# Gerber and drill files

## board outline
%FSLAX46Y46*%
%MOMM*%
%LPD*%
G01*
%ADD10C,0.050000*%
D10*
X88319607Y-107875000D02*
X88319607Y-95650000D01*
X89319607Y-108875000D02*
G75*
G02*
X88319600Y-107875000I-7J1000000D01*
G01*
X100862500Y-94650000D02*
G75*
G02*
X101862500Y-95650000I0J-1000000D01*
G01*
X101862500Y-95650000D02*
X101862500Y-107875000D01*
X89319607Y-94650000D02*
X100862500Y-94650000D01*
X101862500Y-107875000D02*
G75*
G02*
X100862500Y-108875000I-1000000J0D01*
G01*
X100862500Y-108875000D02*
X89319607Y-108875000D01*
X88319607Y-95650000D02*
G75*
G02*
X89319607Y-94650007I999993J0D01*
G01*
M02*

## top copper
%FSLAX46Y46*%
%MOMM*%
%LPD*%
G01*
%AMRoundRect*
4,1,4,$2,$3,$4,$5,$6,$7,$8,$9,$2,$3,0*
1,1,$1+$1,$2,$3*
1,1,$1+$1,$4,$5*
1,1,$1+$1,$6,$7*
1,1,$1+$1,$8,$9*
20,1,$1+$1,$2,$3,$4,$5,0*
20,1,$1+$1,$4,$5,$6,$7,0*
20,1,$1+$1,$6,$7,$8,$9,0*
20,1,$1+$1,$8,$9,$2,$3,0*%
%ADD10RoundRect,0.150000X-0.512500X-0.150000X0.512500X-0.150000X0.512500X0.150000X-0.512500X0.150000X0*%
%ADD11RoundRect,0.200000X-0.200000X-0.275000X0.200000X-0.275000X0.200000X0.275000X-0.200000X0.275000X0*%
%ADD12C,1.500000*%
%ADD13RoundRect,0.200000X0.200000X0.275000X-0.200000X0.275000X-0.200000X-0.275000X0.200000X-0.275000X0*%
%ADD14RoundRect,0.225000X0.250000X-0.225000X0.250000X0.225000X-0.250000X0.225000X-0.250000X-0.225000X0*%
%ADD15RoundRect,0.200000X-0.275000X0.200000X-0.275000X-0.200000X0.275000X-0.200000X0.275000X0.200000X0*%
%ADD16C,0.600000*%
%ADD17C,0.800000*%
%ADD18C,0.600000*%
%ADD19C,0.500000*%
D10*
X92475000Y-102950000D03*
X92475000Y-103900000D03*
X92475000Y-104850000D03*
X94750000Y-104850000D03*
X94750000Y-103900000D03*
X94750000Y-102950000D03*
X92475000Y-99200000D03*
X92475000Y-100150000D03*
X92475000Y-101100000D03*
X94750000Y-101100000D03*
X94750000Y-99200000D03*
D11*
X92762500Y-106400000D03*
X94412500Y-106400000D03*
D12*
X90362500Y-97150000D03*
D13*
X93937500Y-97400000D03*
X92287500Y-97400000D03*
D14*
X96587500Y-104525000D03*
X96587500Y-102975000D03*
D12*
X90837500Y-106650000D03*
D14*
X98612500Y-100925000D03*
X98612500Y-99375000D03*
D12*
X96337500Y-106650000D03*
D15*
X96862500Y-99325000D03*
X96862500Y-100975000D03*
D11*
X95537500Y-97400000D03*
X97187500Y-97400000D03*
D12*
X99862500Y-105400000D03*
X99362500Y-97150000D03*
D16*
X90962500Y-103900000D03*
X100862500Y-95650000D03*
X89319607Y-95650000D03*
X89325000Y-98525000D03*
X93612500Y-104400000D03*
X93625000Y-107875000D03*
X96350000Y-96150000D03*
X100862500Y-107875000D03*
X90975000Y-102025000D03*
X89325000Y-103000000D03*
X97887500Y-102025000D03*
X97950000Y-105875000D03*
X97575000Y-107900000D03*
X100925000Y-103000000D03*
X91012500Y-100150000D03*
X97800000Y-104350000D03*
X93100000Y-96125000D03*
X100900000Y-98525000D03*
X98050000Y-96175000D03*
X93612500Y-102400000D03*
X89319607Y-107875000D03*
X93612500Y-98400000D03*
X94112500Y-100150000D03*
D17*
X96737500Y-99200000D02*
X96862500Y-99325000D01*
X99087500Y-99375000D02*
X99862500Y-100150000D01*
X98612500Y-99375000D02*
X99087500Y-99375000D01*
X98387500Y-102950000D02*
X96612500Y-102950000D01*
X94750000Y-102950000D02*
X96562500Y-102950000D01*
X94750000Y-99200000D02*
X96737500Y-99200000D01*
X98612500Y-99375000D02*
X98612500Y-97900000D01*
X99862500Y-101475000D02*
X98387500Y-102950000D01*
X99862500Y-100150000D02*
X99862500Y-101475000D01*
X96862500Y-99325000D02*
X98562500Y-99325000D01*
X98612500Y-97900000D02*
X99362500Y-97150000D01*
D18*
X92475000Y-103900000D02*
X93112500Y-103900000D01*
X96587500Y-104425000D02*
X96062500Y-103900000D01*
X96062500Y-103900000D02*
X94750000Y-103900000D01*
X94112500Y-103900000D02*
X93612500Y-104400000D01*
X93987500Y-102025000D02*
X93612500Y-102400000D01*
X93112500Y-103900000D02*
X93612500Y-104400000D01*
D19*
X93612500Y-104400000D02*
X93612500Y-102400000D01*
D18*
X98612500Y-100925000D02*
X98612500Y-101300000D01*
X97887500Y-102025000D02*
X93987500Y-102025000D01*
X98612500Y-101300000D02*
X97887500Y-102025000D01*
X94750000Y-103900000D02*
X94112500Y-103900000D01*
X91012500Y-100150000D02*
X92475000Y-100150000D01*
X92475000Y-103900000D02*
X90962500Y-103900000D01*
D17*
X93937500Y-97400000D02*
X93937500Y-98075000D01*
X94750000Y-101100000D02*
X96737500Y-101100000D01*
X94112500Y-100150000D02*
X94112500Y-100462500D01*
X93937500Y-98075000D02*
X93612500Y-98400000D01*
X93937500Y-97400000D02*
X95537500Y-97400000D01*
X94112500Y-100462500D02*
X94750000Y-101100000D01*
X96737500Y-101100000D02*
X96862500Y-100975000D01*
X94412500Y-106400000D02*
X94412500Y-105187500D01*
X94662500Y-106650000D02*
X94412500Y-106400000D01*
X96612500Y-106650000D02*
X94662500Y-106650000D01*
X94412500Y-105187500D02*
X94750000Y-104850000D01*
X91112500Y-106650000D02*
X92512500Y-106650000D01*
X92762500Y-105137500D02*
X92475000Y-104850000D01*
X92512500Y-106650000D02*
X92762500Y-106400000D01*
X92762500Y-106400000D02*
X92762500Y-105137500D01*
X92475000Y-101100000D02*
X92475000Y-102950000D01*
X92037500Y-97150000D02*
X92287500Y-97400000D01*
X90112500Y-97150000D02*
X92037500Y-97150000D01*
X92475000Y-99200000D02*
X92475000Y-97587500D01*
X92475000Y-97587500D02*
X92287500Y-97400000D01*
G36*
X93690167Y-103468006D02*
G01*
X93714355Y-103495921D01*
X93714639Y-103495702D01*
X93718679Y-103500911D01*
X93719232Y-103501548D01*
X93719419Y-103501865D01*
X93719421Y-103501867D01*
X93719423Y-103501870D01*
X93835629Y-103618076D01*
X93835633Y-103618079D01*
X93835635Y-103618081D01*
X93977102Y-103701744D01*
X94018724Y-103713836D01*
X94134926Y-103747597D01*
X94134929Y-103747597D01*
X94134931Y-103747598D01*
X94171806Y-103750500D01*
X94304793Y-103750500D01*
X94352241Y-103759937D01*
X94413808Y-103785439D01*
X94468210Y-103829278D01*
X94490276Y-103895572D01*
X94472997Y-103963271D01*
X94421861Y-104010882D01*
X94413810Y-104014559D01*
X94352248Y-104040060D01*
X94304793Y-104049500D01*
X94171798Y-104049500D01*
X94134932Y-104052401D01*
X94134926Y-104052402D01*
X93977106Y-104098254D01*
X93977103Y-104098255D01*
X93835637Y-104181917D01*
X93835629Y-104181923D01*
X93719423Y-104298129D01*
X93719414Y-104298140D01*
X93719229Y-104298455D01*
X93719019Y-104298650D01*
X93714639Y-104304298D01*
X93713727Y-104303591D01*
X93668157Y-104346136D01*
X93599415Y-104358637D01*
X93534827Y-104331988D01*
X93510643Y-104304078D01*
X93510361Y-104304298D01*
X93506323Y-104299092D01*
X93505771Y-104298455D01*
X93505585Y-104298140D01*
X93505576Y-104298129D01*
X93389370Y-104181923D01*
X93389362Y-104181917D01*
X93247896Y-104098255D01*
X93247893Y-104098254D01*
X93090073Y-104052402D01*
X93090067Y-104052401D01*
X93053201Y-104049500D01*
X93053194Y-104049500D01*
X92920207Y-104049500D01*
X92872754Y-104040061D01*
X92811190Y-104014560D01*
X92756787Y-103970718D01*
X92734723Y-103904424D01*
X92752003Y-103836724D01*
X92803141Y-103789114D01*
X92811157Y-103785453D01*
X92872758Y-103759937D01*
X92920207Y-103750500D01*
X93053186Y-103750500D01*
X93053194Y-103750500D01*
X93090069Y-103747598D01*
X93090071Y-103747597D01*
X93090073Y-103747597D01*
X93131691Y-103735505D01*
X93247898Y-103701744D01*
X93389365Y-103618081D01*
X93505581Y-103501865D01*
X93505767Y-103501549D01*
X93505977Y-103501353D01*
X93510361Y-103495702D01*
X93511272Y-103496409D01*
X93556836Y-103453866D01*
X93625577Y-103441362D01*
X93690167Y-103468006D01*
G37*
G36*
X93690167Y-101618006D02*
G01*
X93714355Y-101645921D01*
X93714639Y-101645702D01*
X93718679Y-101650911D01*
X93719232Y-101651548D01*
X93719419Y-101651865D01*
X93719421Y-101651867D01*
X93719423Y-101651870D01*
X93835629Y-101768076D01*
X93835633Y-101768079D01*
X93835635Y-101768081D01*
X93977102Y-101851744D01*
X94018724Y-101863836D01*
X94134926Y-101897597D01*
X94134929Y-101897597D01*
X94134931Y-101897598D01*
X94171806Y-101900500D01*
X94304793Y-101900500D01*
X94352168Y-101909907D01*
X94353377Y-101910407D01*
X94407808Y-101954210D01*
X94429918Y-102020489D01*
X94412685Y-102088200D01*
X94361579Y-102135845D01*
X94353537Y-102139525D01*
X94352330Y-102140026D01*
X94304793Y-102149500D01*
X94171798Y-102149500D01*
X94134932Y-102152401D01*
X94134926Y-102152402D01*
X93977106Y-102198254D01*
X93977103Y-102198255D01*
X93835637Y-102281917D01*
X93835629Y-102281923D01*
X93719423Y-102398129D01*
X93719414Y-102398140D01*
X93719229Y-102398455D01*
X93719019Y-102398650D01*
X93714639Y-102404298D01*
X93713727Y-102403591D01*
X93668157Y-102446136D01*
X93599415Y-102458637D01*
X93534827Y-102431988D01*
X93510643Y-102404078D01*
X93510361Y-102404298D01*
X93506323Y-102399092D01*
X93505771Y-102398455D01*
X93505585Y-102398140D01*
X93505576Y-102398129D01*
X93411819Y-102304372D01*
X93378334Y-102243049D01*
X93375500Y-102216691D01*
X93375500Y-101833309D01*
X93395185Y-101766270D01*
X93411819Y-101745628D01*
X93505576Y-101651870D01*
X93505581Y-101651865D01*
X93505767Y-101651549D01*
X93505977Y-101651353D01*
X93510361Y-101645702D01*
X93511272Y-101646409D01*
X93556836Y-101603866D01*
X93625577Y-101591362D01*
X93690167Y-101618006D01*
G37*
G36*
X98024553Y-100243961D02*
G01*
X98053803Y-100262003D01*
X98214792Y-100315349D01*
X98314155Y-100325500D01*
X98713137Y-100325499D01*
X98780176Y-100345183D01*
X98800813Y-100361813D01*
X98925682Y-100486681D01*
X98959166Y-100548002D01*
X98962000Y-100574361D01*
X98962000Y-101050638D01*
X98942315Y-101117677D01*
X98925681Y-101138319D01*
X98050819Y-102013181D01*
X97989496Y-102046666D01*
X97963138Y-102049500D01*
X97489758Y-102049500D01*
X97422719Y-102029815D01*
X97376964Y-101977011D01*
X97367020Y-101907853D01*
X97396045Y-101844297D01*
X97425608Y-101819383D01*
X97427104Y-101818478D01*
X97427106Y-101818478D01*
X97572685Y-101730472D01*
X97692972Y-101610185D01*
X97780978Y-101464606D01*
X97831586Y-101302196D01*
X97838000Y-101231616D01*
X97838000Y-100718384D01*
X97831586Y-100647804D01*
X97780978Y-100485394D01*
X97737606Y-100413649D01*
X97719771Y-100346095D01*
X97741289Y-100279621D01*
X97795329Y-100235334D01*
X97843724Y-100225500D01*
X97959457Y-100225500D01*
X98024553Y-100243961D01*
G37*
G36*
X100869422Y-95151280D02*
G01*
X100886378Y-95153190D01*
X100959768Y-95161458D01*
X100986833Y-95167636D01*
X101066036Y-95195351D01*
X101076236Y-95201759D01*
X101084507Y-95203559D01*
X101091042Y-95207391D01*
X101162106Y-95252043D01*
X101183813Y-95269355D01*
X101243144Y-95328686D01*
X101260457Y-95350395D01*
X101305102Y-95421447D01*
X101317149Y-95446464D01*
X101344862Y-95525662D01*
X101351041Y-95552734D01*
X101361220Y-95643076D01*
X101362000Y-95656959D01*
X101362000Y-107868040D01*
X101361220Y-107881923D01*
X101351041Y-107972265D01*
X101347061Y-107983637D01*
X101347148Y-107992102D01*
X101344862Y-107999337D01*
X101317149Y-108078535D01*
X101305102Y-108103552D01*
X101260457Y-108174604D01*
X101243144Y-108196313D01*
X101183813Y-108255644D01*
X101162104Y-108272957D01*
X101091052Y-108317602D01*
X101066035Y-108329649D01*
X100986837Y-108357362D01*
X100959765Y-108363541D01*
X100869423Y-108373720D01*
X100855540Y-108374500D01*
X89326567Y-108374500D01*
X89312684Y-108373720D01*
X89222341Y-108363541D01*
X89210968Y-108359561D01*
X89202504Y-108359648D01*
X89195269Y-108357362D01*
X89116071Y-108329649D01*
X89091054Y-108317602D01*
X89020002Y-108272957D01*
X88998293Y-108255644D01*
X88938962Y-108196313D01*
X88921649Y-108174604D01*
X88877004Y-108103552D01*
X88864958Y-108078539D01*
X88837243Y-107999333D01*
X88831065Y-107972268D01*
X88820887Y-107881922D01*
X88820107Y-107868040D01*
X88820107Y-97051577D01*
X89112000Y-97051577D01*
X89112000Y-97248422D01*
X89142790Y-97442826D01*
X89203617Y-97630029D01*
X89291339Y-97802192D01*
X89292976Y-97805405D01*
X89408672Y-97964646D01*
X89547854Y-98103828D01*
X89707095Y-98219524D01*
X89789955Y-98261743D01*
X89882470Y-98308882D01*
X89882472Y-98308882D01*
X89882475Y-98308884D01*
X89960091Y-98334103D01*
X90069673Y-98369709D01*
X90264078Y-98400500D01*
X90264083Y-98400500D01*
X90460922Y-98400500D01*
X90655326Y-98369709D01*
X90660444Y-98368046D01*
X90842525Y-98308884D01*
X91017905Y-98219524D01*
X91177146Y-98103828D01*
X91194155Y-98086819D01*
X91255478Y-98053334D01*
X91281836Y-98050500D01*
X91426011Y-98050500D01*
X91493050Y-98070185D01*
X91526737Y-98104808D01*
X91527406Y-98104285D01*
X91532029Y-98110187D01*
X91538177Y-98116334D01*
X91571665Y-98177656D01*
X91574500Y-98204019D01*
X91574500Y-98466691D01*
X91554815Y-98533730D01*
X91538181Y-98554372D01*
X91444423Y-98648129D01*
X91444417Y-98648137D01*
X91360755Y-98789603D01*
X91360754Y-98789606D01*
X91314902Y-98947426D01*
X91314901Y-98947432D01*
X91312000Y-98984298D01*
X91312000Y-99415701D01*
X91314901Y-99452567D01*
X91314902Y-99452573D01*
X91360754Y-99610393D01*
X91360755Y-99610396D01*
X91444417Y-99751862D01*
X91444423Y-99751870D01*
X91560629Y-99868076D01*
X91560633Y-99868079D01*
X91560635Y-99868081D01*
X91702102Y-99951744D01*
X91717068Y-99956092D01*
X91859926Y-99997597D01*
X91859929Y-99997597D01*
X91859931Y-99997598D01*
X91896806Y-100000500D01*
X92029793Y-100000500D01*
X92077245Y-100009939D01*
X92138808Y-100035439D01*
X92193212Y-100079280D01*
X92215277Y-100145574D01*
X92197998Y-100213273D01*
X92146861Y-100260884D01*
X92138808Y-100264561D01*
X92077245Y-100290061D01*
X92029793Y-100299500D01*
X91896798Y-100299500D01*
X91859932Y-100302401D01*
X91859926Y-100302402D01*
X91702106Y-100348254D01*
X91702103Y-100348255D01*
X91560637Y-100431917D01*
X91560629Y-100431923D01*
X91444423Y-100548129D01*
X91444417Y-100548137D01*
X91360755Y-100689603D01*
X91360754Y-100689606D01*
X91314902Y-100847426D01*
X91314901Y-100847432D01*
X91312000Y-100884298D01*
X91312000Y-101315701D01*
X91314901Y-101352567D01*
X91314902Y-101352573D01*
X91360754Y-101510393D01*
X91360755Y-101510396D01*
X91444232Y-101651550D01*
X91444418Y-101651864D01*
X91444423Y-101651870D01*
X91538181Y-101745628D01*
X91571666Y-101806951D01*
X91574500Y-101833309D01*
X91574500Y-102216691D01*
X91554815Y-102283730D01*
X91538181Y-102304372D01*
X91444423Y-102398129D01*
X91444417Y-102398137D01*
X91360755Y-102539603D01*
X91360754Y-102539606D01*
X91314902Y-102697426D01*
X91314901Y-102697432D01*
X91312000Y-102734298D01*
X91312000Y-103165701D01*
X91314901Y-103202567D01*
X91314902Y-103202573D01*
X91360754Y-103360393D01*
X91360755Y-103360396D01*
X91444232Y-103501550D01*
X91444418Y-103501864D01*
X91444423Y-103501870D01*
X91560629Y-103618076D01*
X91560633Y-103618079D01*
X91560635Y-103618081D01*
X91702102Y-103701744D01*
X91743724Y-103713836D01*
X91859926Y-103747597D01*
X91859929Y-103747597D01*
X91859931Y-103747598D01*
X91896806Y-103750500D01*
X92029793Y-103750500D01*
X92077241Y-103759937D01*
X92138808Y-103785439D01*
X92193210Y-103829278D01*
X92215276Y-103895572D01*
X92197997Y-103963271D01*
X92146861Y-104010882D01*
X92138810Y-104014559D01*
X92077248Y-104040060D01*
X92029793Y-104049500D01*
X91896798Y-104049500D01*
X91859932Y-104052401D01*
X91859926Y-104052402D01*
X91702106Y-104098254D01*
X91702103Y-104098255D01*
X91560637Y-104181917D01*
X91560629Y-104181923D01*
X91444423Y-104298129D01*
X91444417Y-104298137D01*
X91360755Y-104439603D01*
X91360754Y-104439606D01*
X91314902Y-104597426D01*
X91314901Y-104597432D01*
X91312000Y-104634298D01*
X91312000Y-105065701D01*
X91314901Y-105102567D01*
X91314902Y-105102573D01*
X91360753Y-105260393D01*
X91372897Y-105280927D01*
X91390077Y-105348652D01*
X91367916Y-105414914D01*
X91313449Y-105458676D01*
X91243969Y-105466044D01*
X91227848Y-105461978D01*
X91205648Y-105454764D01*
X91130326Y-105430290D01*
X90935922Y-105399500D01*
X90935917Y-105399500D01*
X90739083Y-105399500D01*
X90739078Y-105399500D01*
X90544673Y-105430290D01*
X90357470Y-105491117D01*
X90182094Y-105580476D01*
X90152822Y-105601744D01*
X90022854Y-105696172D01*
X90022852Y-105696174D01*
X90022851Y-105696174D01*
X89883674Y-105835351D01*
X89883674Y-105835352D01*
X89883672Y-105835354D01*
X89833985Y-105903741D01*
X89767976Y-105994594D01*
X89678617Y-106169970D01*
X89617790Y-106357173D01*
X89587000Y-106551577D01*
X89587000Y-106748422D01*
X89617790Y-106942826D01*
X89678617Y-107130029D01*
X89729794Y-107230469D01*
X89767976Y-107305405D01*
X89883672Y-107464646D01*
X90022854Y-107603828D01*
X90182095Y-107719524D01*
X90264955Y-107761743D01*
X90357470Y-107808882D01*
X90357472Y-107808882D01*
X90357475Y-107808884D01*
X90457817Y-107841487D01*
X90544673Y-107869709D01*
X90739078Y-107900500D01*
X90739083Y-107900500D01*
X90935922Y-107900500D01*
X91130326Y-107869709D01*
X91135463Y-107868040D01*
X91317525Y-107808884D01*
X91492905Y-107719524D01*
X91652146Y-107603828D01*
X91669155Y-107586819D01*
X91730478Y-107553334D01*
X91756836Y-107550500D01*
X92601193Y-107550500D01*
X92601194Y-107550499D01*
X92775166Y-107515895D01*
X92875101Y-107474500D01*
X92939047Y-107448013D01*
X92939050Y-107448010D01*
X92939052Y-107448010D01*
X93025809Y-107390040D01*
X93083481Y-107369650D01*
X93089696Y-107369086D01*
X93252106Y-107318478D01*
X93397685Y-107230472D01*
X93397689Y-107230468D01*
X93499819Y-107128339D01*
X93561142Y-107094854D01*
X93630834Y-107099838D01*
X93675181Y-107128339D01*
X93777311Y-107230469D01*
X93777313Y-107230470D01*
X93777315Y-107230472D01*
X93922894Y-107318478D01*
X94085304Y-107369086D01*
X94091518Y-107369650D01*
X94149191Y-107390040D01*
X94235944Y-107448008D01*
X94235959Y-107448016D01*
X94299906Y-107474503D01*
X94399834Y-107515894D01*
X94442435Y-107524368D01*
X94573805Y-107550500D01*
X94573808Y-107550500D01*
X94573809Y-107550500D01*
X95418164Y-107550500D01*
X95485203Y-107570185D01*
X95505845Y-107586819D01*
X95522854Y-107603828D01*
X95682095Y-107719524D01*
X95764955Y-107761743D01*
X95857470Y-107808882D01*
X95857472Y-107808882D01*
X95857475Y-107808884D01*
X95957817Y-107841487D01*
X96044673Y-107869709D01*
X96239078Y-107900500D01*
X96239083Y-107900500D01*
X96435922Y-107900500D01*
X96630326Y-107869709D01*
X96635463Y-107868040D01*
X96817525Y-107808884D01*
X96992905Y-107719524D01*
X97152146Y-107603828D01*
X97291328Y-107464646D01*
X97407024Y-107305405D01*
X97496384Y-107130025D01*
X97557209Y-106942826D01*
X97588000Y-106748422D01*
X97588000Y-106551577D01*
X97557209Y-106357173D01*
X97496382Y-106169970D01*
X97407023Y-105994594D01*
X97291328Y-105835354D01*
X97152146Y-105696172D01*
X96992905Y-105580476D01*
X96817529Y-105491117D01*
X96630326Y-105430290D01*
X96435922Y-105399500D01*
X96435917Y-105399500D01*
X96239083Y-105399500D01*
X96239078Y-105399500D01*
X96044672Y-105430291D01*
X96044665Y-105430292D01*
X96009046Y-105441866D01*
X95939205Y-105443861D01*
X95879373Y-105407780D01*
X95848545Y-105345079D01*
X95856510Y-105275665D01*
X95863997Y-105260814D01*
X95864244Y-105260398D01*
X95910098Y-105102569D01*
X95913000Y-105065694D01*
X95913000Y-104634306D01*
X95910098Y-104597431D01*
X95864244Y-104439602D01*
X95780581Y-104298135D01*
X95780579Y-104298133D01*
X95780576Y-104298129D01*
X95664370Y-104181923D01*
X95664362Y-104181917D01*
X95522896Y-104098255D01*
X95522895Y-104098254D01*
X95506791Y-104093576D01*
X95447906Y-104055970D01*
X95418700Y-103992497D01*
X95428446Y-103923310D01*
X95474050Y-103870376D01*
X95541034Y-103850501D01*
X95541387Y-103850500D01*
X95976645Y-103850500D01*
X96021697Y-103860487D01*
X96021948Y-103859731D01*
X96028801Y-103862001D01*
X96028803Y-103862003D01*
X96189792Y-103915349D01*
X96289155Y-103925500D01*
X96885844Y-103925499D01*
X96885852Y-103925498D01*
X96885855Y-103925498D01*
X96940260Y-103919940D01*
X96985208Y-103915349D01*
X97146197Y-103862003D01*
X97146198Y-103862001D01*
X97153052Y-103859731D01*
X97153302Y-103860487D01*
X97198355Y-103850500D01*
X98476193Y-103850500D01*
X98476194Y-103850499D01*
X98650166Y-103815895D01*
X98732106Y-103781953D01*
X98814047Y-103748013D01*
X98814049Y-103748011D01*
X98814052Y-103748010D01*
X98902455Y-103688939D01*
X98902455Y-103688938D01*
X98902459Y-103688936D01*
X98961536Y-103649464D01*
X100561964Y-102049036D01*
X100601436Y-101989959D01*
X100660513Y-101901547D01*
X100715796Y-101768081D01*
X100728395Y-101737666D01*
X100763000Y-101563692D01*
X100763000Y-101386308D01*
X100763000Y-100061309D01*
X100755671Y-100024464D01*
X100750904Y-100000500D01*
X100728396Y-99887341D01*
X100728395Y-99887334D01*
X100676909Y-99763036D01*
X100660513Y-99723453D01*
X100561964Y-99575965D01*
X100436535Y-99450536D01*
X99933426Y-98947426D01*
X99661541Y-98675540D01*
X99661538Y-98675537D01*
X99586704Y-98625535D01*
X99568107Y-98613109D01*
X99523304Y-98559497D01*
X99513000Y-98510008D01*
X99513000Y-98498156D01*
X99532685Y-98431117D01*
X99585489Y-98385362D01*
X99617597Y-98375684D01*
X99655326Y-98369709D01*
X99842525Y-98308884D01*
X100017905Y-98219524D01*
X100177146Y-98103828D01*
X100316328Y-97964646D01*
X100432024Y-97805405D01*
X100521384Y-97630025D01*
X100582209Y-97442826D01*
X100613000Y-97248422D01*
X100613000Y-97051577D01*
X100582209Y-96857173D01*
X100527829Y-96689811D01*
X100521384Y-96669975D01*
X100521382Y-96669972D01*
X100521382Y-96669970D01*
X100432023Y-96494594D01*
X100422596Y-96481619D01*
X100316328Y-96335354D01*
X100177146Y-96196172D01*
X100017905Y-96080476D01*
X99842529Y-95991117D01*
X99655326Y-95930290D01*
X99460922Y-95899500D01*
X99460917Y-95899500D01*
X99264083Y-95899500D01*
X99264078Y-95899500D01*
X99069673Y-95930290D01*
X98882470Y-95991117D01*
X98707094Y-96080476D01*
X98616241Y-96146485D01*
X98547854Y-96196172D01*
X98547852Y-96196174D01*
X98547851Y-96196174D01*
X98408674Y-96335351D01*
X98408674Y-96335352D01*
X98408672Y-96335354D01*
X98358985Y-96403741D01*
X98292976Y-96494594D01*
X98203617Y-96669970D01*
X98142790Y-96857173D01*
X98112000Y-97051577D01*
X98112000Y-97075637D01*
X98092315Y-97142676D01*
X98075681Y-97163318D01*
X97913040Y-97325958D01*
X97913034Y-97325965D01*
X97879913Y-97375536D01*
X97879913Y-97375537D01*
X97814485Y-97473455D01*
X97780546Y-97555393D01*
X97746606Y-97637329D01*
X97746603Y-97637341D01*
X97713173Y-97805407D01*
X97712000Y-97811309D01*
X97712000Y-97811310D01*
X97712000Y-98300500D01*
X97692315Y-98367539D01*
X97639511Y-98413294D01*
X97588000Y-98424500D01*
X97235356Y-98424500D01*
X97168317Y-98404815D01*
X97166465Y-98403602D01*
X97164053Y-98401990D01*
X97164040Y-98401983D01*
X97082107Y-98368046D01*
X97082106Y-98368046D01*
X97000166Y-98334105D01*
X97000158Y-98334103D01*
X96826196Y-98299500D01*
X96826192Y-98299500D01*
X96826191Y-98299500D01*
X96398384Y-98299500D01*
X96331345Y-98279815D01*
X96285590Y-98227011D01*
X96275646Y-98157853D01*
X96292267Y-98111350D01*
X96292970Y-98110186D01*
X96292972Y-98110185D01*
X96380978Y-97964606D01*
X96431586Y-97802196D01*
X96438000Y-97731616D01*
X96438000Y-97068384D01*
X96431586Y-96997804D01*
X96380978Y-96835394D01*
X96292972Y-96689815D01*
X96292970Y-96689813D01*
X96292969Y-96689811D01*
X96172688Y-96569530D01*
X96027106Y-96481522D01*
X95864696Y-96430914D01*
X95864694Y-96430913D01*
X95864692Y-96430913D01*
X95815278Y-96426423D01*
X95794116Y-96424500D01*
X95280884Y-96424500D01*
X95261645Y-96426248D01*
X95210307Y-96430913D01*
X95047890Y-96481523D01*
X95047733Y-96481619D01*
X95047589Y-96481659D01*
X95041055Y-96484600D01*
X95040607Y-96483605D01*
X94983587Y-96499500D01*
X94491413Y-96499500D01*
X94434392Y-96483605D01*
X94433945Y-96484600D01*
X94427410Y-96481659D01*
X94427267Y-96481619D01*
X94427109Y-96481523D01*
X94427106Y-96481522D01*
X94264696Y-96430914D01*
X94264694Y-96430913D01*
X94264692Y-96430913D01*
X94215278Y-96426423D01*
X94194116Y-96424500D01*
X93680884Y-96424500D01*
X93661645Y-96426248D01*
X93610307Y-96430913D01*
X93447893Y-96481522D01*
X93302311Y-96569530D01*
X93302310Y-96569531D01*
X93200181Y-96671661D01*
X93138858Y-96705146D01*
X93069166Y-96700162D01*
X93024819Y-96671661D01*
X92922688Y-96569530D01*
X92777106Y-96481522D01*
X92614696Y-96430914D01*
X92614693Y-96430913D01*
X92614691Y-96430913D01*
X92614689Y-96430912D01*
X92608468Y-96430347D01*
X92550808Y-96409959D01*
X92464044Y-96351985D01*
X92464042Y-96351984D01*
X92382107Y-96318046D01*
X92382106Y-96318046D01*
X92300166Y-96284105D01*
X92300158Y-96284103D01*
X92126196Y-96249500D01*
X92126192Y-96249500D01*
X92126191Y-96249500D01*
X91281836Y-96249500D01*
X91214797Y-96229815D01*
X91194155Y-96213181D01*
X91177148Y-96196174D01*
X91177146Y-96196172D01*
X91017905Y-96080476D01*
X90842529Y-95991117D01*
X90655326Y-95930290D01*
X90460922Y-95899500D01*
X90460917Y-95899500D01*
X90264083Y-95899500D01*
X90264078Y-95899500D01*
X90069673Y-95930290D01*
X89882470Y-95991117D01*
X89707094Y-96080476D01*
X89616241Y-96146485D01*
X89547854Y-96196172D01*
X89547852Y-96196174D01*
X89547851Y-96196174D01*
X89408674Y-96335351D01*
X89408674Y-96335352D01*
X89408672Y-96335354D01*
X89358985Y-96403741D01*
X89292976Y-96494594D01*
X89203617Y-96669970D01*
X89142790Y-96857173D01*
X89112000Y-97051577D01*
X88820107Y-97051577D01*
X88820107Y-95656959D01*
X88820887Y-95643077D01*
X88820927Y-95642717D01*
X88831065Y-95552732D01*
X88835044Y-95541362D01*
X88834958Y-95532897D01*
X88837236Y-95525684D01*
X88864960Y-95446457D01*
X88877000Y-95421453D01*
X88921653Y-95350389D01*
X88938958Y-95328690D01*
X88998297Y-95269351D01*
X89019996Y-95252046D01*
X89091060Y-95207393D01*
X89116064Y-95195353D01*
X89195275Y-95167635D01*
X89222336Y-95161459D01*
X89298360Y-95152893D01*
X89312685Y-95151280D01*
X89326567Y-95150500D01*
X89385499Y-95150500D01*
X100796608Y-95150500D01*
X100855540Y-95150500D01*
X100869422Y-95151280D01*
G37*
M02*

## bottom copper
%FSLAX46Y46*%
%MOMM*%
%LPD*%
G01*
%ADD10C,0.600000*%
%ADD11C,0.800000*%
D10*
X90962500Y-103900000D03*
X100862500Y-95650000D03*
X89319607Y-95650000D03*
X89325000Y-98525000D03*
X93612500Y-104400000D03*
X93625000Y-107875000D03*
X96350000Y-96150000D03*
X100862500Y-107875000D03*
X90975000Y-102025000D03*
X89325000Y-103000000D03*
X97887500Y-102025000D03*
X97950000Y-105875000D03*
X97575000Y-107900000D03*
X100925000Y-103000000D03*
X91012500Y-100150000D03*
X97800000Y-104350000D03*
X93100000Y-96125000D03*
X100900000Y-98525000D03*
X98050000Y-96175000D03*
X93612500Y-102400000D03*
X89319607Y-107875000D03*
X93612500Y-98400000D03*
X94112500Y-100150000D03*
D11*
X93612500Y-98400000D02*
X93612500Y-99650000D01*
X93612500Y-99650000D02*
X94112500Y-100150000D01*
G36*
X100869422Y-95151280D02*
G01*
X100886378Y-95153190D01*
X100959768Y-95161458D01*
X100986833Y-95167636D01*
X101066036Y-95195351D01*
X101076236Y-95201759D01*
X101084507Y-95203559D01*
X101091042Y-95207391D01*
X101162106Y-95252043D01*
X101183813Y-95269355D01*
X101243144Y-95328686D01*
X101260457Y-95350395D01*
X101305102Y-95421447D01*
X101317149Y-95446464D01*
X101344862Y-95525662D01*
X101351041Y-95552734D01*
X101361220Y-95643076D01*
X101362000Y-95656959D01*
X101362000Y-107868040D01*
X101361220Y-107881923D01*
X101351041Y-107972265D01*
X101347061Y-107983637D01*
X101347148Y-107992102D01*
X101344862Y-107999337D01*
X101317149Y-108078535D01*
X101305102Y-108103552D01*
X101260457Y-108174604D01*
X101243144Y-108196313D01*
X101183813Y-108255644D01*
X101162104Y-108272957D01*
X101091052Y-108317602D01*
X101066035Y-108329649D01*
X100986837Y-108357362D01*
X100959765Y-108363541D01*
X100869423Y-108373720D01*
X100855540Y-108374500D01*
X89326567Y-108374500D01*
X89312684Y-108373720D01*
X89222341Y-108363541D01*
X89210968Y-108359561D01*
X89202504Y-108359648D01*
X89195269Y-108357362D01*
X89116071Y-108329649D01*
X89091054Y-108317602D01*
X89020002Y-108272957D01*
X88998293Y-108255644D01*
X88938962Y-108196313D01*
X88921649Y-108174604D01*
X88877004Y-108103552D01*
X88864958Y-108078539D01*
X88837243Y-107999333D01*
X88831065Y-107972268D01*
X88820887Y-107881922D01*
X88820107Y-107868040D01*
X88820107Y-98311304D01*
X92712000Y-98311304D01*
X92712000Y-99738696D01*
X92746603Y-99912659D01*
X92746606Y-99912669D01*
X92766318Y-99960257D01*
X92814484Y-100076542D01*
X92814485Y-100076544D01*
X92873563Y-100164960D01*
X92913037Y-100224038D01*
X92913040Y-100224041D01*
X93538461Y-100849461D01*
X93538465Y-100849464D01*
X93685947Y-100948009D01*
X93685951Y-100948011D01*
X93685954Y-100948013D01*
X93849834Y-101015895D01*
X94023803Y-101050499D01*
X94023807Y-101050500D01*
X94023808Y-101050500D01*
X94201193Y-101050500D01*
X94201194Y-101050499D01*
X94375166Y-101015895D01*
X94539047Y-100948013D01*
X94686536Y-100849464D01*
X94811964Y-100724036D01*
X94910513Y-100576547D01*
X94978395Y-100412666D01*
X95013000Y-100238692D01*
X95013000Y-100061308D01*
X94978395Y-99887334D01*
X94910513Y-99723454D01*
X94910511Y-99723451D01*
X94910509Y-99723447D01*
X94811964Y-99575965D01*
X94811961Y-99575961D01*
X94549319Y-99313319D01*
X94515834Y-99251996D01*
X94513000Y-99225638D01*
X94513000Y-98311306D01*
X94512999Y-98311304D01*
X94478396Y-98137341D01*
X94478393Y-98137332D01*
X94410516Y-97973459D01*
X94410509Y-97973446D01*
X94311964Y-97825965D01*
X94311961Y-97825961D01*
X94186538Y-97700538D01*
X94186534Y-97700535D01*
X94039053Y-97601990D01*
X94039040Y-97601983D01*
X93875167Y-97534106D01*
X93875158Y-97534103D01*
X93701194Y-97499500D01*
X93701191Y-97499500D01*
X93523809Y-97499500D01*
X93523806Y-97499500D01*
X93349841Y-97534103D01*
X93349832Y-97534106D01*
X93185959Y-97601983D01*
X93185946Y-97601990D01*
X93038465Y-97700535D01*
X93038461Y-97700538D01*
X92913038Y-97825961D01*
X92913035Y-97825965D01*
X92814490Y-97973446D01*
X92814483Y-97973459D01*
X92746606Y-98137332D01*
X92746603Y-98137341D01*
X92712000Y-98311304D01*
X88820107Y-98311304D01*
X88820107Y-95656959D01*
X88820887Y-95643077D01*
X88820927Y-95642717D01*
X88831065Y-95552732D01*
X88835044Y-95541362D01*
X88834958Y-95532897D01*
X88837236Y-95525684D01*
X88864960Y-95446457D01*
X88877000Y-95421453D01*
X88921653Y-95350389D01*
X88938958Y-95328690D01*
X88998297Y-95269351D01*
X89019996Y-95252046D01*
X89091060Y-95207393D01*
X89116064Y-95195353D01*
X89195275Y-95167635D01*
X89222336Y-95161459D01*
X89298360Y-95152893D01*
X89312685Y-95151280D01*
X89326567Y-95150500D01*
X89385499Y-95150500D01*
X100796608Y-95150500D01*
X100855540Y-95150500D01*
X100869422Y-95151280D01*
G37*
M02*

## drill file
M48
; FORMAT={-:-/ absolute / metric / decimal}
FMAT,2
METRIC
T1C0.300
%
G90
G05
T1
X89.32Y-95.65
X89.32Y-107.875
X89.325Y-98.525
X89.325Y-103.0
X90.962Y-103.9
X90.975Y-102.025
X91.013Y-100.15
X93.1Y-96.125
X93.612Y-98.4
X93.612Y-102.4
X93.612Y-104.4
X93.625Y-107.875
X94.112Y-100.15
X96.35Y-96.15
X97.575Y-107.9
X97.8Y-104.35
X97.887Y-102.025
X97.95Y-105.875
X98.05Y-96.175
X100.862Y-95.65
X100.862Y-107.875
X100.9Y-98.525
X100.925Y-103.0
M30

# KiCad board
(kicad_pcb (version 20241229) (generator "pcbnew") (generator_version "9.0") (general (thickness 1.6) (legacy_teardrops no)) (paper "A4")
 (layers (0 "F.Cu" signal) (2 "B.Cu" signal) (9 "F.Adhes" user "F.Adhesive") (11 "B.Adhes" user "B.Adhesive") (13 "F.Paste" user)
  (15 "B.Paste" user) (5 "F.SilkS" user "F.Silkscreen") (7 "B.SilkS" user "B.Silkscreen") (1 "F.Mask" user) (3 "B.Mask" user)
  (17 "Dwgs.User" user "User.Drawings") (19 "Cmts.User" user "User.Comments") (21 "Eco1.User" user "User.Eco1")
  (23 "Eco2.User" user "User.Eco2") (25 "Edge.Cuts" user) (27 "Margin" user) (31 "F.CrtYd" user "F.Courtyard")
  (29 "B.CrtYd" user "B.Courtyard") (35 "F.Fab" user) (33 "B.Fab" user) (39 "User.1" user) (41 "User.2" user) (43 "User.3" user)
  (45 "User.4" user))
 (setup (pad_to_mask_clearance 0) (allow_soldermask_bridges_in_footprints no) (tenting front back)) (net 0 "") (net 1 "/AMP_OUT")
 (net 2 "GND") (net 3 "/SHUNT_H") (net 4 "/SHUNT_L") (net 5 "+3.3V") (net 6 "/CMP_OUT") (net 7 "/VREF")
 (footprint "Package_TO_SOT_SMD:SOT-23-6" (layer "F.Cu") (at 93.6125 103.9)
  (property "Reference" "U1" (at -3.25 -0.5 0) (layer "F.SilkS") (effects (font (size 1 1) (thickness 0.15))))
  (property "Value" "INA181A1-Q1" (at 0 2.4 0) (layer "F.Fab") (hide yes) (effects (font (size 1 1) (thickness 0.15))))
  (pad "1" smd roundrect (at -1.1375 -0.95) (size 1.325 0.6) (layers "F.Cu" "F.Mask" "F.Paste") (roundrect_rratio 0.25) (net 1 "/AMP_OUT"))
  (pad "2" smd roundrect (at -1.1375 0) (size 1.325 0.6) (layers "F.Cu" "F.Mask" "F.Paste") (roundrect_rratio 0.25) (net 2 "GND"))
  (pad "3" smd roundrect (at -1.1375 0.95) (size 1.325 0.6) (layers "F.Cu" "F.Mask" "F.Paste") (roundrect_rratio 0.25) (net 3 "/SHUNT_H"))
  (pad "4" smd roundrect (at 1.1375 0.95) (size 1.325 0.6) (layers "F.Cu" "F.Mask" "F.Paste") (roundrect_rratio 0.25) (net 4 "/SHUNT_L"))
  (pad "5" smd roundrect (at 1.1375 0) (size 1.325 0.6) (layers "F.Cu" "F.Mask" "F.Paste") (roundrect_rratio 0.25) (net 2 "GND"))
  (pad "6" smd roundrect (at 1.1375 -0.95) (size 1.325 0.6) (layers "F.Cu" "F.Mask" "F.Paste") (roundrect_rratio 0.25) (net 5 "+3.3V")))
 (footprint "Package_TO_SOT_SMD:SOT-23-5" (layer "F.Cu") (at 93.6125 100.15)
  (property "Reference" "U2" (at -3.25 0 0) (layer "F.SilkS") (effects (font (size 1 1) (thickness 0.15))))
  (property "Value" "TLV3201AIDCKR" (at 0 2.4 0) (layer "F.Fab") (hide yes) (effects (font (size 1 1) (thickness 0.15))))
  (pad "1" smd roundrect (at -1.1375 -0.95) (size 1.325 0.6) (layers "F.Cu" "F.Mask" "F.Paste") (roundrect_rratio 0.25) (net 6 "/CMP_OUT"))
  (pad "2" smd roundrect (at -1.1375 0) (size 1.325 0.6) (layers "F.Cu" "F.Mask" "F.Paste") (roundrect_rratio 0.25) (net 2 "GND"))
  (pad "3" smd roundrect (at -1.1375 0.95) (size 1.325 0.6) (layers "F.Cu" "F.Mask" "F.Paste") (roundrect_rratio 0.25) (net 1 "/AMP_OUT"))
  (pad "4" smd roundrect (at 1.1375 0.95) (size 1.325 0.6) (layers "F.Cu" "F.Mask" "F.Paste") (roundrect_rratio 0.25) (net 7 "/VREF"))
  (pad "5" smd roundrect (at 1.1375 -0.95) (size 1.325 0.6) (layers "F.Cu" "F.Mask" "F.Paste") (roundrect_rratio 0.25) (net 5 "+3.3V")))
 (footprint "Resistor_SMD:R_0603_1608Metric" (layer "F.Cu") (at 93.5875 106.4)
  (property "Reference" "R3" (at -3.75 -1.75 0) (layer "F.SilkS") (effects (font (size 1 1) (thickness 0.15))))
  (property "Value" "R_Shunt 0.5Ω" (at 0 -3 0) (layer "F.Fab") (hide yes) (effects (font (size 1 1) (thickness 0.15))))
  (pad "1" smd roundrect (at -0.825 0) (size 0.8 0.95) (layers "F.Cu" "F.Mask" "F.Paste") (roundrect_rratio 0.25) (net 3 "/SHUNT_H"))
  (pad "2" smd roundrect (at 0.825 0) (size 0.8 0.95) (layers "F.Cu" "F.Mask" "F.Paste") (roundrect_rratio 0.25) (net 4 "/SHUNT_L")))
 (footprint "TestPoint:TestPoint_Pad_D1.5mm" (layer "F.Cu") (at 90.3625 97.15)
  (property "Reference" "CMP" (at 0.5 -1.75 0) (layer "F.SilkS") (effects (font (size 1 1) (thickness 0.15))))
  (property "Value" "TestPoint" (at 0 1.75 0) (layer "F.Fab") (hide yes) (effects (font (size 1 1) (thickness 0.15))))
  (pad "1" smd circle (at 0 0) (size 1.5 1.5) (layers "F.Cu" "F.Mask") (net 6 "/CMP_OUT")))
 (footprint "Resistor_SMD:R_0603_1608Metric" (layer "F.Cu") (at 93.1125 97.4 180)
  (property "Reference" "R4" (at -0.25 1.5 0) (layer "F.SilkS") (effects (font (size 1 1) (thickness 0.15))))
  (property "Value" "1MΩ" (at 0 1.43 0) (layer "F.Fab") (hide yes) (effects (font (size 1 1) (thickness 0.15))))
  (pad "1" smd roundrect (at -0.825 0 180) (size 0.8 0.95) (layers "F.Cu" "F.Mask" "F.Paste") (roundrect_rratio 0.25) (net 7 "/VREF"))
  (pad "2" smd roundrect (at 0.825 0 180) (size 0.8 0.95) (layers "F.Cu" "F.Mask" "F.Paste") (roundrect_rratio 0.25) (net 6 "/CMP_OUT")))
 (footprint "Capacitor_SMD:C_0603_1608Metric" (layer "F.Cu") (at 96.5875 103.75 90)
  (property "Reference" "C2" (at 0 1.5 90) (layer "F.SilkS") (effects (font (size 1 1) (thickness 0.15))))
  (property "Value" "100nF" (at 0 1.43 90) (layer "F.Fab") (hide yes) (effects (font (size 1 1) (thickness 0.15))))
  (pad "1" smd roundrect (at -0.775 0 90) (size 0.9 0.95) (layers "F.Cu" "F.Mask" "F.Paste") (roundrect_rratio 0.25) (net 2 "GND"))
  (pad "2" smd roundrect (at 0.775 0 90) (size 0.9 0.95) (layers "F.Cu" "F.Mask" "F.Paste") (roundrect_rratio 0.25) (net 5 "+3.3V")))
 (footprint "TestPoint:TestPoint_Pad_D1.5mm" (layer "F.Cu") (at 90.8375 106.65)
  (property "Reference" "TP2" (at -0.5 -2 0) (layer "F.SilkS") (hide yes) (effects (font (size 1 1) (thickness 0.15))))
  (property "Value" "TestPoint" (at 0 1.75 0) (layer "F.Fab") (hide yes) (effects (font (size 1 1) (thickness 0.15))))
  (pad "1" smd circle (at 0 0) (size 1.5 1.5) (layers "F.Cu" "F.Mask") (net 3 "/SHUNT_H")))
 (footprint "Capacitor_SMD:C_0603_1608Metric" (layer "F.Cu") (at 98.6125 100.15 90)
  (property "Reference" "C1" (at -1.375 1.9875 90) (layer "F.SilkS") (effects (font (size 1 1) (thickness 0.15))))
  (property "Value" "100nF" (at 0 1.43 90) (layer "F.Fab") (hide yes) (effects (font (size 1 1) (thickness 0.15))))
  (pad "1" smd roundrect (at -0.775 0 90) (size 0.9 0.95) (layers "F.Cu" "F.Mask" "F.Paste") (roundrect_rratio 0.25) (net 2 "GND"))
  (pad "2" smd roundrect (at 0.775 0 90) (size 0.9 0.95) (layers "F.Cu" "F.Mask" "F.Paste") (roundrect_rratio 0.25) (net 5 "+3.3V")))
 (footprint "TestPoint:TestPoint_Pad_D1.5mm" (layer "F.Cu") (at 96.3375 106.65)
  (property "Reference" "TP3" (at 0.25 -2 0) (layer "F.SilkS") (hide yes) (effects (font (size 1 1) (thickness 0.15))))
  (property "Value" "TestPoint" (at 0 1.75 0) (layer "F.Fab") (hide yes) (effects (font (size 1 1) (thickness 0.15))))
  (pad "1" smd circle (at 0 0) (size 1.5 1.5) (layers "F.Cu" "F.Mask") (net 4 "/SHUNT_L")))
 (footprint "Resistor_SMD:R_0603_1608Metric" (layer "F.Cu") (at 96.8625 100.15 -90)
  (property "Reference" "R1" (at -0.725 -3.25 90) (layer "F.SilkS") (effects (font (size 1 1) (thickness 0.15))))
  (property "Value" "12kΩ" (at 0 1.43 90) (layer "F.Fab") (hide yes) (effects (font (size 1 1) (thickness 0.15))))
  (pad "1" smd roundrect (at -0.825 0 270) (size 0.8 0.95) (layers "F.Cu" "F.Mask" "F.Paste") (roundrect_rratio 0.25) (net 5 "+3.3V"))
  (pad "2" smd roundrect (at 0.825 0 270) (size 0.8 0.95) (layers "F.Cu" "F.Mask" "F.Paste") (roundrect_rratio 0.25) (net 7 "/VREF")))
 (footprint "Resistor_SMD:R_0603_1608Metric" (layer "F.Cu") (at 96.3625 97.4)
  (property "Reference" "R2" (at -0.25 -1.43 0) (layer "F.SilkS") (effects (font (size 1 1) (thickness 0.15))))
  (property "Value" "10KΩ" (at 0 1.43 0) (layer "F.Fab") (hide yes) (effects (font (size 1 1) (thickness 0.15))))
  (pad "1" smd roundrect (at -0.825 0) (size 0.8 0.95) (layers "F.Cu" "F.Mask" "F.Paste") (roundrect_rratio 0.25) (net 7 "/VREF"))
  (pad "2" smd roundrect (at 0.825 0) (size 0.8 0.95) (layers "F.Cu" "F.Mask" "F.Paste") (roundrect_rratio 0.25) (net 2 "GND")))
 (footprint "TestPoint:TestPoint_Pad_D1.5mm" (layer "F.Cu") (at 99.8625 105.4)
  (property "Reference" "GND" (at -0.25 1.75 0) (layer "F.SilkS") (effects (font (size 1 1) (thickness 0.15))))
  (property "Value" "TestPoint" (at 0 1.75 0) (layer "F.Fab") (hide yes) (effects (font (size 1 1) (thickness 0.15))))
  (pad "1" smd circle (at 0 0) (size 1.5 1.5) (layers "F.Cu" "F.Mask") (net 2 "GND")))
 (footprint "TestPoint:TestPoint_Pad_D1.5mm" (layer "F.Cu") (at 99.3625 97.15)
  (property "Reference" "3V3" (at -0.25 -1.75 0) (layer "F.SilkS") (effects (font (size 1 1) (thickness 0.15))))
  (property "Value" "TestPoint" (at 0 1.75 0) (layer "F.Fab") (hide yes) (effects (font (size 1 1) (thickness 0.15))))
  (pad "1" smd circle (at 0 0) (size 1.5 1.5) (layers "F.Cu" "F.Mask") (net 5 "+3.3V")))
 (gr_line (start 88.319607 107.875) (end 88.319607 95.65) (stroke (width 0.05) (type default)) (layer "Edge.Cuts"))
 (gr_arc (start 89.319607 108.875) (mid 88.6125 108.582107) (end 88.319607 107.875) (stroke (width 0.05) (type default)) (layer "Edge.Cuts"))
 (gr_arc (start 100.8625 94.65) (mid 101.569607 94.942893) (end 101.8625 95.65) (stroke (width 0.05) (type default)) (layer "Edge.Cuts"))
 (gr_line (start 101.8625 95.65) (end 101.8625 107.875) (stroke (width 0.05) (type default)) (layer "Edge.Cuts"))
 (gr_line (start 89.319607 94.65) (end 100.8625 94.65) (stroke (width 0.05) (type default)) (layer "Edge.Cuts"))
 (gr_arc (start 101.8625 107.875) (mid 101.569607 108.582107) (end 100.8625 108.875) (stroke (width 0.05) (type default))
  (layer "Edge.Cuts"))
 (gr_line (start 100.8625 108.875) (end 89.319607 108.875) (stroke (width 0.05) (type default)) (layer "Edge.Cuts"))
 (gr_arc (start 88.319607 95.65) (mid 88.6125 94.942893) (end 89.319607 94.65) (stroke (width 0.05) (type default)) (layer "Edge.Cuts"))
 (segment (start 96.7375 99.2) (end 96.8625 99.325) (width 0.8) (layer "F.Cu") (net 5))
 (segment (start 99.0875 99.375) (end 99.8625 100.15) (width 0.8) (layer "F.Cu") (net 5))
 (segment (start 98.6125 99.375) (end 99.0875 99.375) (width 0.8) (layer "F.Cu") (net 5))
 (segment (start 98.3875 102.95) (end 96.6125 102.95) (width 0.8) (layer "F.Cu") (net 5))
 (segment (start 94.75 102.95) (end 96.5625 102.95) (width 0.8) (layer "F.Cu") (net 5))
 (segment (start 94.75 99.2) (end 96.7375 99.2) (width 0.8) (layer "F.Cu") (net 5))
 (segment (start 98.6125 99.375) (end 98.6125 97.9) (width 0.8) (layer "F.Cu") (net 5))
 (segment (start 99.8625 101.475) (end 98.3875 102.95) (width 0.8) (layer "F.Cu") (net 5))
 (segment (start 99.8625 100.15) (end 99.8625 101.475) (width 0.8) (layer "F.Cu") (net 5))
 (segment (start 96.8625 99.325) (end 98.5625 99.325) (width 0.8) (layer "F.Cu") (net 5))
 (segment (start 98.6125 97.9) (end 99.3625 97.15) (width 0.8) (layer "F.Cu") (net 5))
 (segment (start 92.475 103.9) (end 93.1125 103.9) (width 0.6) (layer "F.Cu") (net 2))
 (segment (start 96.5875 104.425) (end 96.0625 103.9) (width 0.6) (layer "F.Cu") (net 2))
 (segment (start 96.0625 103.9) (end 94.75 103.9) (width 0.6) (layer "F.Cu") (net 2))
 (segment (start 94.1125 103.9) (end 93.6125 104.4) (width 0.6) (layer "F.Cu") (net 2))
 (segment (start 93.9875 102.025) (end 93.6125 102.4) (width 0.6) (layer "F.Cu") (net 2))
 (segment (start 93.1125 103.9) (end 93.6125 104.4) (width 0.6) (layer "F.Cu") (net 2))
 (segment (start 93.6125 104.4) (end 93.6125 102.4) (width 0.5) (layer "F.Cu") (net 2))
 (segment (start 98.6125 100.925) (end 98.6125 101.3) (width 0.6) (layer "F.Cu") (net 2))
 (segment (start 97.8875 102.025) (end 93.9875 102.025) (width 0.6) (layer "F.Cu") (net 2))
 (segment (start 98.6125 101.3) (end 97.8875 102.025) (width 0.6) (layer "F.Cu") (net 2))
 (segment (start 94.75 103.9) (end 94.1125 103.9) (width 0.6) (layer "F.Cu") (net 2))
 (segment (start 91.0125 100.15) (end 92.475 100.15) (width 0.6) (layer "F.Cu") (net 2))
 (segment (start 92.475 103.9) (end 90.9625 103.9) (width 0.6) (layer "F.Cu") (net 2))
 (via (at 90.9625 103.9) (size 0.6) (drill 0.3) (layers "F.Cu" "B.Cu") (free yes) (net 2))
 (via (at 100.8625 95.65) (size 0.6) (drill 0.3) (layers "F.Cu" "B.Cu") (free yes) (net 2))
 (via (at 89.319607 95.65) (size 0.6) (drill 0.3) (layers "F.Cu" "B.Cu") (free yes) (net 2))
 (via (at 89.325 98.525) (size 0.6) (drill 0.3) (layers "F.Cu" "B.Cu") (free yes) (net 2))
 (via (at 93.6125 104.4) (size 0.6) (drill 0.3) (layers "F.Cu" "B.Cu") (free yes) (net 2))
 (via (at 93.625 107.875) (size 0.6) (drill 0.3) (layers "F.Cu" "B.Cu") (free yes) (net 2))
 (via (at 96.35 96.15) (size 0.6) (drill 0.3) (layers "F.Cu" "B.Cu") (free yes) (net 2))
 (via (at 100.8625 107.875) (size 0.6) (drill 0.3) (layers "F.Cu" "B.Cu") (free yes) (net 2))
 (via (at 90.975 102.025) (size 0.6) (drill 0.3) (layers "F.Cu" "B.Cu") (free yes) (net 2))
 (via (at 89.325 103) (size 0.6) (drill 0.3) (layers "F.Cu" "B.Cu") (free yes) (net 2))
 (via (at 97.8875 102.025) (size 0.6) (drill 0.3) (layers "F.Cu" "B.Cu") (free yes) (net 2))
 (via (at 97.95 105.875) (size 0.6) (drill 0.3) (layers "F.Cu" "B.Cu") (free yes) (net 2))
 (via (at 97.575 107.9) (size 0.6) (drill 0.3) (layers "F.Cu" "B.Cu") (free yes) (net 2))
 (via (at 100.925 103) (size 0.6) (drill 0.3) (layers "F.Cu" "B.Cu") (free yes) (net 2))
 (via (at 91.0125 100.15) (size 0.6) (drill 0.3) (layers "F.Cu" "B.Cu") (free yes) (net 2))
 (via (at 97.8 104.35) (size 0.6) (drill 0.3) (layers "F.Cu" "B.Cu") (free yes) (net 2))
 (via (at 93.1 96.125) (size 0.6) (drill 0.3) (layers "F.Cu" "B.Cu") (free yes) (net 2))
 (via (at 100.9 98.525) (size 0.6) (drill 0.3) (layers "F.Cu" "B.Cu") (free yes) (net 2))
 (via (at 98.05 96.175) (size 0.6) (drill 0.3) (layers "F.Cu" "B.Cu") (free yes) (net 2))
 (via (at 93.6125 102.4) (size 0.6) (drill 0.3) (layers "F.Cu" "B.Cu") (free yes) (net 2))
 (via (at 89.319607 107.875) (size 0.6) (drill 0.3) (layers "F.Cu" "B.Cu") (free yes) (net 2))
 (segment (start 93.9375 97.4) (end 93.9375 98.075) (width 0.8) (layer "F.Cu") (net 7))
 (segment (start 94.75 101.1) (end 96.7375 101.1) (width 0.8) (layer "F.Cu") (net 7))
 (segment (start 94.1125 100.15) (end 94.1125 100.4625) (width 0.8) (layer "F.Cu") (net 7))
 (segment (start 93.9375 98.075) (end 93.6125 98.4) (width 0.8) (layer "F.Cu") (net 7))
 (segment (start 93.9375 97.4) (end 95.5375 97.4) (width 0.8) (layer "F.Cu") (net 7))
 (segment (start 94.1125 100.4625) (end 94.75 101.1) (width 0.8) (layer "F.Cu") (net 7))
 (segment (start 96.7375 101.1) (end 96.8625 100.975) (width 0.8) (layer "F.Cu") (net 7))
 (via (at 93.6125 98.4) (size 0.6) (drill 0.3) (layers "F.Cu" "B.Cu") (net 7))
 (via (at 94.1125 100.15) (size 0.6) (drill 0.3) (layers "F.Cu" "B.Cu") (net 7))
 (segment (start 93.6125 98.4) (end 93.6125 99.65) (width 0.8) (layer "B.Cu") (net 7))
 (segment (start 93.6125 99.65) (end 94.1125 100.15) (width 0.8) (layer "B.Cu") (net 7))
 (segment (start 94.4125 106.4) (end 94.4125 105.1875) (width 0.8) (layer "F.Cu") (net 4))
 (segment (start 94.6625 106.65) (end 94.4125 106.4) (width 0.8) (layer "F.Cu") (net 4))
 (segment (start 96.6125 106.65) (end 94.6625 106.65) (width 0.8) (layer "F.Cu") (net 4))
 (segment (start 94.4125 105.1875) (end 94.75 104.85) (width 0.8) (layer "F.Cu") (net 4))
 (segment (start 91.1125 106.65) (end 92.5125 106.65) (width 0.8) (layer "F.Cu") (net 3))
 (segment (start 92.7625 105.1375) (end 92.475 104.85) (width 0.8) (layer "F.Cu") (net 3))
 (segment (start 92.5125 106.65) (end 92.7625 106.4) (width 0.8) (layer "F.Cu") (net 3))
 (segment (start 92.7625 106.4) (end 92.7625 105.1375) (width 0.8) (layer "F.Cu") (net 3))
 (segment (start 92.475 101.1) (end 92.475 102.95) (width 0.8) (layer "F.Cu") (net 1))
 (segment (start 92.0375 97.15) (end 92.2875 97.4) (width 0.8) (layer "F.Cu") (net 6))
 (segment (start 90.1125 97.15) (end 92.0375 97.15) (width 0.8) (layer "F.Cu") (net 6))
 (segment (start 92.475 99.2) (end 92.475 97.5875) (width 0.8) (layer "F.Cu") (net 6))
 (segment (start 92.475 97.5875) (end 92.2875 97.4) (width 0.8) (layer "F.Cu") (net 6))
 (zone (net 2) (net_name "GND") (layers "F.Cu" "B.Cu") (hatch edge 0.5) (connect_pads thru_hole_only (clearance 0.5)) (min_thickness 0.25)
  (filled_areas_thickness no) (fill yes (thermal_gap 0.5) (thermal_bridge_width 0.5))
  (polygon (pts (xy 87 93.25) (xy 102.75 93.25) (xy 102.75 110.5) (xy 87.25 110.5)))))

